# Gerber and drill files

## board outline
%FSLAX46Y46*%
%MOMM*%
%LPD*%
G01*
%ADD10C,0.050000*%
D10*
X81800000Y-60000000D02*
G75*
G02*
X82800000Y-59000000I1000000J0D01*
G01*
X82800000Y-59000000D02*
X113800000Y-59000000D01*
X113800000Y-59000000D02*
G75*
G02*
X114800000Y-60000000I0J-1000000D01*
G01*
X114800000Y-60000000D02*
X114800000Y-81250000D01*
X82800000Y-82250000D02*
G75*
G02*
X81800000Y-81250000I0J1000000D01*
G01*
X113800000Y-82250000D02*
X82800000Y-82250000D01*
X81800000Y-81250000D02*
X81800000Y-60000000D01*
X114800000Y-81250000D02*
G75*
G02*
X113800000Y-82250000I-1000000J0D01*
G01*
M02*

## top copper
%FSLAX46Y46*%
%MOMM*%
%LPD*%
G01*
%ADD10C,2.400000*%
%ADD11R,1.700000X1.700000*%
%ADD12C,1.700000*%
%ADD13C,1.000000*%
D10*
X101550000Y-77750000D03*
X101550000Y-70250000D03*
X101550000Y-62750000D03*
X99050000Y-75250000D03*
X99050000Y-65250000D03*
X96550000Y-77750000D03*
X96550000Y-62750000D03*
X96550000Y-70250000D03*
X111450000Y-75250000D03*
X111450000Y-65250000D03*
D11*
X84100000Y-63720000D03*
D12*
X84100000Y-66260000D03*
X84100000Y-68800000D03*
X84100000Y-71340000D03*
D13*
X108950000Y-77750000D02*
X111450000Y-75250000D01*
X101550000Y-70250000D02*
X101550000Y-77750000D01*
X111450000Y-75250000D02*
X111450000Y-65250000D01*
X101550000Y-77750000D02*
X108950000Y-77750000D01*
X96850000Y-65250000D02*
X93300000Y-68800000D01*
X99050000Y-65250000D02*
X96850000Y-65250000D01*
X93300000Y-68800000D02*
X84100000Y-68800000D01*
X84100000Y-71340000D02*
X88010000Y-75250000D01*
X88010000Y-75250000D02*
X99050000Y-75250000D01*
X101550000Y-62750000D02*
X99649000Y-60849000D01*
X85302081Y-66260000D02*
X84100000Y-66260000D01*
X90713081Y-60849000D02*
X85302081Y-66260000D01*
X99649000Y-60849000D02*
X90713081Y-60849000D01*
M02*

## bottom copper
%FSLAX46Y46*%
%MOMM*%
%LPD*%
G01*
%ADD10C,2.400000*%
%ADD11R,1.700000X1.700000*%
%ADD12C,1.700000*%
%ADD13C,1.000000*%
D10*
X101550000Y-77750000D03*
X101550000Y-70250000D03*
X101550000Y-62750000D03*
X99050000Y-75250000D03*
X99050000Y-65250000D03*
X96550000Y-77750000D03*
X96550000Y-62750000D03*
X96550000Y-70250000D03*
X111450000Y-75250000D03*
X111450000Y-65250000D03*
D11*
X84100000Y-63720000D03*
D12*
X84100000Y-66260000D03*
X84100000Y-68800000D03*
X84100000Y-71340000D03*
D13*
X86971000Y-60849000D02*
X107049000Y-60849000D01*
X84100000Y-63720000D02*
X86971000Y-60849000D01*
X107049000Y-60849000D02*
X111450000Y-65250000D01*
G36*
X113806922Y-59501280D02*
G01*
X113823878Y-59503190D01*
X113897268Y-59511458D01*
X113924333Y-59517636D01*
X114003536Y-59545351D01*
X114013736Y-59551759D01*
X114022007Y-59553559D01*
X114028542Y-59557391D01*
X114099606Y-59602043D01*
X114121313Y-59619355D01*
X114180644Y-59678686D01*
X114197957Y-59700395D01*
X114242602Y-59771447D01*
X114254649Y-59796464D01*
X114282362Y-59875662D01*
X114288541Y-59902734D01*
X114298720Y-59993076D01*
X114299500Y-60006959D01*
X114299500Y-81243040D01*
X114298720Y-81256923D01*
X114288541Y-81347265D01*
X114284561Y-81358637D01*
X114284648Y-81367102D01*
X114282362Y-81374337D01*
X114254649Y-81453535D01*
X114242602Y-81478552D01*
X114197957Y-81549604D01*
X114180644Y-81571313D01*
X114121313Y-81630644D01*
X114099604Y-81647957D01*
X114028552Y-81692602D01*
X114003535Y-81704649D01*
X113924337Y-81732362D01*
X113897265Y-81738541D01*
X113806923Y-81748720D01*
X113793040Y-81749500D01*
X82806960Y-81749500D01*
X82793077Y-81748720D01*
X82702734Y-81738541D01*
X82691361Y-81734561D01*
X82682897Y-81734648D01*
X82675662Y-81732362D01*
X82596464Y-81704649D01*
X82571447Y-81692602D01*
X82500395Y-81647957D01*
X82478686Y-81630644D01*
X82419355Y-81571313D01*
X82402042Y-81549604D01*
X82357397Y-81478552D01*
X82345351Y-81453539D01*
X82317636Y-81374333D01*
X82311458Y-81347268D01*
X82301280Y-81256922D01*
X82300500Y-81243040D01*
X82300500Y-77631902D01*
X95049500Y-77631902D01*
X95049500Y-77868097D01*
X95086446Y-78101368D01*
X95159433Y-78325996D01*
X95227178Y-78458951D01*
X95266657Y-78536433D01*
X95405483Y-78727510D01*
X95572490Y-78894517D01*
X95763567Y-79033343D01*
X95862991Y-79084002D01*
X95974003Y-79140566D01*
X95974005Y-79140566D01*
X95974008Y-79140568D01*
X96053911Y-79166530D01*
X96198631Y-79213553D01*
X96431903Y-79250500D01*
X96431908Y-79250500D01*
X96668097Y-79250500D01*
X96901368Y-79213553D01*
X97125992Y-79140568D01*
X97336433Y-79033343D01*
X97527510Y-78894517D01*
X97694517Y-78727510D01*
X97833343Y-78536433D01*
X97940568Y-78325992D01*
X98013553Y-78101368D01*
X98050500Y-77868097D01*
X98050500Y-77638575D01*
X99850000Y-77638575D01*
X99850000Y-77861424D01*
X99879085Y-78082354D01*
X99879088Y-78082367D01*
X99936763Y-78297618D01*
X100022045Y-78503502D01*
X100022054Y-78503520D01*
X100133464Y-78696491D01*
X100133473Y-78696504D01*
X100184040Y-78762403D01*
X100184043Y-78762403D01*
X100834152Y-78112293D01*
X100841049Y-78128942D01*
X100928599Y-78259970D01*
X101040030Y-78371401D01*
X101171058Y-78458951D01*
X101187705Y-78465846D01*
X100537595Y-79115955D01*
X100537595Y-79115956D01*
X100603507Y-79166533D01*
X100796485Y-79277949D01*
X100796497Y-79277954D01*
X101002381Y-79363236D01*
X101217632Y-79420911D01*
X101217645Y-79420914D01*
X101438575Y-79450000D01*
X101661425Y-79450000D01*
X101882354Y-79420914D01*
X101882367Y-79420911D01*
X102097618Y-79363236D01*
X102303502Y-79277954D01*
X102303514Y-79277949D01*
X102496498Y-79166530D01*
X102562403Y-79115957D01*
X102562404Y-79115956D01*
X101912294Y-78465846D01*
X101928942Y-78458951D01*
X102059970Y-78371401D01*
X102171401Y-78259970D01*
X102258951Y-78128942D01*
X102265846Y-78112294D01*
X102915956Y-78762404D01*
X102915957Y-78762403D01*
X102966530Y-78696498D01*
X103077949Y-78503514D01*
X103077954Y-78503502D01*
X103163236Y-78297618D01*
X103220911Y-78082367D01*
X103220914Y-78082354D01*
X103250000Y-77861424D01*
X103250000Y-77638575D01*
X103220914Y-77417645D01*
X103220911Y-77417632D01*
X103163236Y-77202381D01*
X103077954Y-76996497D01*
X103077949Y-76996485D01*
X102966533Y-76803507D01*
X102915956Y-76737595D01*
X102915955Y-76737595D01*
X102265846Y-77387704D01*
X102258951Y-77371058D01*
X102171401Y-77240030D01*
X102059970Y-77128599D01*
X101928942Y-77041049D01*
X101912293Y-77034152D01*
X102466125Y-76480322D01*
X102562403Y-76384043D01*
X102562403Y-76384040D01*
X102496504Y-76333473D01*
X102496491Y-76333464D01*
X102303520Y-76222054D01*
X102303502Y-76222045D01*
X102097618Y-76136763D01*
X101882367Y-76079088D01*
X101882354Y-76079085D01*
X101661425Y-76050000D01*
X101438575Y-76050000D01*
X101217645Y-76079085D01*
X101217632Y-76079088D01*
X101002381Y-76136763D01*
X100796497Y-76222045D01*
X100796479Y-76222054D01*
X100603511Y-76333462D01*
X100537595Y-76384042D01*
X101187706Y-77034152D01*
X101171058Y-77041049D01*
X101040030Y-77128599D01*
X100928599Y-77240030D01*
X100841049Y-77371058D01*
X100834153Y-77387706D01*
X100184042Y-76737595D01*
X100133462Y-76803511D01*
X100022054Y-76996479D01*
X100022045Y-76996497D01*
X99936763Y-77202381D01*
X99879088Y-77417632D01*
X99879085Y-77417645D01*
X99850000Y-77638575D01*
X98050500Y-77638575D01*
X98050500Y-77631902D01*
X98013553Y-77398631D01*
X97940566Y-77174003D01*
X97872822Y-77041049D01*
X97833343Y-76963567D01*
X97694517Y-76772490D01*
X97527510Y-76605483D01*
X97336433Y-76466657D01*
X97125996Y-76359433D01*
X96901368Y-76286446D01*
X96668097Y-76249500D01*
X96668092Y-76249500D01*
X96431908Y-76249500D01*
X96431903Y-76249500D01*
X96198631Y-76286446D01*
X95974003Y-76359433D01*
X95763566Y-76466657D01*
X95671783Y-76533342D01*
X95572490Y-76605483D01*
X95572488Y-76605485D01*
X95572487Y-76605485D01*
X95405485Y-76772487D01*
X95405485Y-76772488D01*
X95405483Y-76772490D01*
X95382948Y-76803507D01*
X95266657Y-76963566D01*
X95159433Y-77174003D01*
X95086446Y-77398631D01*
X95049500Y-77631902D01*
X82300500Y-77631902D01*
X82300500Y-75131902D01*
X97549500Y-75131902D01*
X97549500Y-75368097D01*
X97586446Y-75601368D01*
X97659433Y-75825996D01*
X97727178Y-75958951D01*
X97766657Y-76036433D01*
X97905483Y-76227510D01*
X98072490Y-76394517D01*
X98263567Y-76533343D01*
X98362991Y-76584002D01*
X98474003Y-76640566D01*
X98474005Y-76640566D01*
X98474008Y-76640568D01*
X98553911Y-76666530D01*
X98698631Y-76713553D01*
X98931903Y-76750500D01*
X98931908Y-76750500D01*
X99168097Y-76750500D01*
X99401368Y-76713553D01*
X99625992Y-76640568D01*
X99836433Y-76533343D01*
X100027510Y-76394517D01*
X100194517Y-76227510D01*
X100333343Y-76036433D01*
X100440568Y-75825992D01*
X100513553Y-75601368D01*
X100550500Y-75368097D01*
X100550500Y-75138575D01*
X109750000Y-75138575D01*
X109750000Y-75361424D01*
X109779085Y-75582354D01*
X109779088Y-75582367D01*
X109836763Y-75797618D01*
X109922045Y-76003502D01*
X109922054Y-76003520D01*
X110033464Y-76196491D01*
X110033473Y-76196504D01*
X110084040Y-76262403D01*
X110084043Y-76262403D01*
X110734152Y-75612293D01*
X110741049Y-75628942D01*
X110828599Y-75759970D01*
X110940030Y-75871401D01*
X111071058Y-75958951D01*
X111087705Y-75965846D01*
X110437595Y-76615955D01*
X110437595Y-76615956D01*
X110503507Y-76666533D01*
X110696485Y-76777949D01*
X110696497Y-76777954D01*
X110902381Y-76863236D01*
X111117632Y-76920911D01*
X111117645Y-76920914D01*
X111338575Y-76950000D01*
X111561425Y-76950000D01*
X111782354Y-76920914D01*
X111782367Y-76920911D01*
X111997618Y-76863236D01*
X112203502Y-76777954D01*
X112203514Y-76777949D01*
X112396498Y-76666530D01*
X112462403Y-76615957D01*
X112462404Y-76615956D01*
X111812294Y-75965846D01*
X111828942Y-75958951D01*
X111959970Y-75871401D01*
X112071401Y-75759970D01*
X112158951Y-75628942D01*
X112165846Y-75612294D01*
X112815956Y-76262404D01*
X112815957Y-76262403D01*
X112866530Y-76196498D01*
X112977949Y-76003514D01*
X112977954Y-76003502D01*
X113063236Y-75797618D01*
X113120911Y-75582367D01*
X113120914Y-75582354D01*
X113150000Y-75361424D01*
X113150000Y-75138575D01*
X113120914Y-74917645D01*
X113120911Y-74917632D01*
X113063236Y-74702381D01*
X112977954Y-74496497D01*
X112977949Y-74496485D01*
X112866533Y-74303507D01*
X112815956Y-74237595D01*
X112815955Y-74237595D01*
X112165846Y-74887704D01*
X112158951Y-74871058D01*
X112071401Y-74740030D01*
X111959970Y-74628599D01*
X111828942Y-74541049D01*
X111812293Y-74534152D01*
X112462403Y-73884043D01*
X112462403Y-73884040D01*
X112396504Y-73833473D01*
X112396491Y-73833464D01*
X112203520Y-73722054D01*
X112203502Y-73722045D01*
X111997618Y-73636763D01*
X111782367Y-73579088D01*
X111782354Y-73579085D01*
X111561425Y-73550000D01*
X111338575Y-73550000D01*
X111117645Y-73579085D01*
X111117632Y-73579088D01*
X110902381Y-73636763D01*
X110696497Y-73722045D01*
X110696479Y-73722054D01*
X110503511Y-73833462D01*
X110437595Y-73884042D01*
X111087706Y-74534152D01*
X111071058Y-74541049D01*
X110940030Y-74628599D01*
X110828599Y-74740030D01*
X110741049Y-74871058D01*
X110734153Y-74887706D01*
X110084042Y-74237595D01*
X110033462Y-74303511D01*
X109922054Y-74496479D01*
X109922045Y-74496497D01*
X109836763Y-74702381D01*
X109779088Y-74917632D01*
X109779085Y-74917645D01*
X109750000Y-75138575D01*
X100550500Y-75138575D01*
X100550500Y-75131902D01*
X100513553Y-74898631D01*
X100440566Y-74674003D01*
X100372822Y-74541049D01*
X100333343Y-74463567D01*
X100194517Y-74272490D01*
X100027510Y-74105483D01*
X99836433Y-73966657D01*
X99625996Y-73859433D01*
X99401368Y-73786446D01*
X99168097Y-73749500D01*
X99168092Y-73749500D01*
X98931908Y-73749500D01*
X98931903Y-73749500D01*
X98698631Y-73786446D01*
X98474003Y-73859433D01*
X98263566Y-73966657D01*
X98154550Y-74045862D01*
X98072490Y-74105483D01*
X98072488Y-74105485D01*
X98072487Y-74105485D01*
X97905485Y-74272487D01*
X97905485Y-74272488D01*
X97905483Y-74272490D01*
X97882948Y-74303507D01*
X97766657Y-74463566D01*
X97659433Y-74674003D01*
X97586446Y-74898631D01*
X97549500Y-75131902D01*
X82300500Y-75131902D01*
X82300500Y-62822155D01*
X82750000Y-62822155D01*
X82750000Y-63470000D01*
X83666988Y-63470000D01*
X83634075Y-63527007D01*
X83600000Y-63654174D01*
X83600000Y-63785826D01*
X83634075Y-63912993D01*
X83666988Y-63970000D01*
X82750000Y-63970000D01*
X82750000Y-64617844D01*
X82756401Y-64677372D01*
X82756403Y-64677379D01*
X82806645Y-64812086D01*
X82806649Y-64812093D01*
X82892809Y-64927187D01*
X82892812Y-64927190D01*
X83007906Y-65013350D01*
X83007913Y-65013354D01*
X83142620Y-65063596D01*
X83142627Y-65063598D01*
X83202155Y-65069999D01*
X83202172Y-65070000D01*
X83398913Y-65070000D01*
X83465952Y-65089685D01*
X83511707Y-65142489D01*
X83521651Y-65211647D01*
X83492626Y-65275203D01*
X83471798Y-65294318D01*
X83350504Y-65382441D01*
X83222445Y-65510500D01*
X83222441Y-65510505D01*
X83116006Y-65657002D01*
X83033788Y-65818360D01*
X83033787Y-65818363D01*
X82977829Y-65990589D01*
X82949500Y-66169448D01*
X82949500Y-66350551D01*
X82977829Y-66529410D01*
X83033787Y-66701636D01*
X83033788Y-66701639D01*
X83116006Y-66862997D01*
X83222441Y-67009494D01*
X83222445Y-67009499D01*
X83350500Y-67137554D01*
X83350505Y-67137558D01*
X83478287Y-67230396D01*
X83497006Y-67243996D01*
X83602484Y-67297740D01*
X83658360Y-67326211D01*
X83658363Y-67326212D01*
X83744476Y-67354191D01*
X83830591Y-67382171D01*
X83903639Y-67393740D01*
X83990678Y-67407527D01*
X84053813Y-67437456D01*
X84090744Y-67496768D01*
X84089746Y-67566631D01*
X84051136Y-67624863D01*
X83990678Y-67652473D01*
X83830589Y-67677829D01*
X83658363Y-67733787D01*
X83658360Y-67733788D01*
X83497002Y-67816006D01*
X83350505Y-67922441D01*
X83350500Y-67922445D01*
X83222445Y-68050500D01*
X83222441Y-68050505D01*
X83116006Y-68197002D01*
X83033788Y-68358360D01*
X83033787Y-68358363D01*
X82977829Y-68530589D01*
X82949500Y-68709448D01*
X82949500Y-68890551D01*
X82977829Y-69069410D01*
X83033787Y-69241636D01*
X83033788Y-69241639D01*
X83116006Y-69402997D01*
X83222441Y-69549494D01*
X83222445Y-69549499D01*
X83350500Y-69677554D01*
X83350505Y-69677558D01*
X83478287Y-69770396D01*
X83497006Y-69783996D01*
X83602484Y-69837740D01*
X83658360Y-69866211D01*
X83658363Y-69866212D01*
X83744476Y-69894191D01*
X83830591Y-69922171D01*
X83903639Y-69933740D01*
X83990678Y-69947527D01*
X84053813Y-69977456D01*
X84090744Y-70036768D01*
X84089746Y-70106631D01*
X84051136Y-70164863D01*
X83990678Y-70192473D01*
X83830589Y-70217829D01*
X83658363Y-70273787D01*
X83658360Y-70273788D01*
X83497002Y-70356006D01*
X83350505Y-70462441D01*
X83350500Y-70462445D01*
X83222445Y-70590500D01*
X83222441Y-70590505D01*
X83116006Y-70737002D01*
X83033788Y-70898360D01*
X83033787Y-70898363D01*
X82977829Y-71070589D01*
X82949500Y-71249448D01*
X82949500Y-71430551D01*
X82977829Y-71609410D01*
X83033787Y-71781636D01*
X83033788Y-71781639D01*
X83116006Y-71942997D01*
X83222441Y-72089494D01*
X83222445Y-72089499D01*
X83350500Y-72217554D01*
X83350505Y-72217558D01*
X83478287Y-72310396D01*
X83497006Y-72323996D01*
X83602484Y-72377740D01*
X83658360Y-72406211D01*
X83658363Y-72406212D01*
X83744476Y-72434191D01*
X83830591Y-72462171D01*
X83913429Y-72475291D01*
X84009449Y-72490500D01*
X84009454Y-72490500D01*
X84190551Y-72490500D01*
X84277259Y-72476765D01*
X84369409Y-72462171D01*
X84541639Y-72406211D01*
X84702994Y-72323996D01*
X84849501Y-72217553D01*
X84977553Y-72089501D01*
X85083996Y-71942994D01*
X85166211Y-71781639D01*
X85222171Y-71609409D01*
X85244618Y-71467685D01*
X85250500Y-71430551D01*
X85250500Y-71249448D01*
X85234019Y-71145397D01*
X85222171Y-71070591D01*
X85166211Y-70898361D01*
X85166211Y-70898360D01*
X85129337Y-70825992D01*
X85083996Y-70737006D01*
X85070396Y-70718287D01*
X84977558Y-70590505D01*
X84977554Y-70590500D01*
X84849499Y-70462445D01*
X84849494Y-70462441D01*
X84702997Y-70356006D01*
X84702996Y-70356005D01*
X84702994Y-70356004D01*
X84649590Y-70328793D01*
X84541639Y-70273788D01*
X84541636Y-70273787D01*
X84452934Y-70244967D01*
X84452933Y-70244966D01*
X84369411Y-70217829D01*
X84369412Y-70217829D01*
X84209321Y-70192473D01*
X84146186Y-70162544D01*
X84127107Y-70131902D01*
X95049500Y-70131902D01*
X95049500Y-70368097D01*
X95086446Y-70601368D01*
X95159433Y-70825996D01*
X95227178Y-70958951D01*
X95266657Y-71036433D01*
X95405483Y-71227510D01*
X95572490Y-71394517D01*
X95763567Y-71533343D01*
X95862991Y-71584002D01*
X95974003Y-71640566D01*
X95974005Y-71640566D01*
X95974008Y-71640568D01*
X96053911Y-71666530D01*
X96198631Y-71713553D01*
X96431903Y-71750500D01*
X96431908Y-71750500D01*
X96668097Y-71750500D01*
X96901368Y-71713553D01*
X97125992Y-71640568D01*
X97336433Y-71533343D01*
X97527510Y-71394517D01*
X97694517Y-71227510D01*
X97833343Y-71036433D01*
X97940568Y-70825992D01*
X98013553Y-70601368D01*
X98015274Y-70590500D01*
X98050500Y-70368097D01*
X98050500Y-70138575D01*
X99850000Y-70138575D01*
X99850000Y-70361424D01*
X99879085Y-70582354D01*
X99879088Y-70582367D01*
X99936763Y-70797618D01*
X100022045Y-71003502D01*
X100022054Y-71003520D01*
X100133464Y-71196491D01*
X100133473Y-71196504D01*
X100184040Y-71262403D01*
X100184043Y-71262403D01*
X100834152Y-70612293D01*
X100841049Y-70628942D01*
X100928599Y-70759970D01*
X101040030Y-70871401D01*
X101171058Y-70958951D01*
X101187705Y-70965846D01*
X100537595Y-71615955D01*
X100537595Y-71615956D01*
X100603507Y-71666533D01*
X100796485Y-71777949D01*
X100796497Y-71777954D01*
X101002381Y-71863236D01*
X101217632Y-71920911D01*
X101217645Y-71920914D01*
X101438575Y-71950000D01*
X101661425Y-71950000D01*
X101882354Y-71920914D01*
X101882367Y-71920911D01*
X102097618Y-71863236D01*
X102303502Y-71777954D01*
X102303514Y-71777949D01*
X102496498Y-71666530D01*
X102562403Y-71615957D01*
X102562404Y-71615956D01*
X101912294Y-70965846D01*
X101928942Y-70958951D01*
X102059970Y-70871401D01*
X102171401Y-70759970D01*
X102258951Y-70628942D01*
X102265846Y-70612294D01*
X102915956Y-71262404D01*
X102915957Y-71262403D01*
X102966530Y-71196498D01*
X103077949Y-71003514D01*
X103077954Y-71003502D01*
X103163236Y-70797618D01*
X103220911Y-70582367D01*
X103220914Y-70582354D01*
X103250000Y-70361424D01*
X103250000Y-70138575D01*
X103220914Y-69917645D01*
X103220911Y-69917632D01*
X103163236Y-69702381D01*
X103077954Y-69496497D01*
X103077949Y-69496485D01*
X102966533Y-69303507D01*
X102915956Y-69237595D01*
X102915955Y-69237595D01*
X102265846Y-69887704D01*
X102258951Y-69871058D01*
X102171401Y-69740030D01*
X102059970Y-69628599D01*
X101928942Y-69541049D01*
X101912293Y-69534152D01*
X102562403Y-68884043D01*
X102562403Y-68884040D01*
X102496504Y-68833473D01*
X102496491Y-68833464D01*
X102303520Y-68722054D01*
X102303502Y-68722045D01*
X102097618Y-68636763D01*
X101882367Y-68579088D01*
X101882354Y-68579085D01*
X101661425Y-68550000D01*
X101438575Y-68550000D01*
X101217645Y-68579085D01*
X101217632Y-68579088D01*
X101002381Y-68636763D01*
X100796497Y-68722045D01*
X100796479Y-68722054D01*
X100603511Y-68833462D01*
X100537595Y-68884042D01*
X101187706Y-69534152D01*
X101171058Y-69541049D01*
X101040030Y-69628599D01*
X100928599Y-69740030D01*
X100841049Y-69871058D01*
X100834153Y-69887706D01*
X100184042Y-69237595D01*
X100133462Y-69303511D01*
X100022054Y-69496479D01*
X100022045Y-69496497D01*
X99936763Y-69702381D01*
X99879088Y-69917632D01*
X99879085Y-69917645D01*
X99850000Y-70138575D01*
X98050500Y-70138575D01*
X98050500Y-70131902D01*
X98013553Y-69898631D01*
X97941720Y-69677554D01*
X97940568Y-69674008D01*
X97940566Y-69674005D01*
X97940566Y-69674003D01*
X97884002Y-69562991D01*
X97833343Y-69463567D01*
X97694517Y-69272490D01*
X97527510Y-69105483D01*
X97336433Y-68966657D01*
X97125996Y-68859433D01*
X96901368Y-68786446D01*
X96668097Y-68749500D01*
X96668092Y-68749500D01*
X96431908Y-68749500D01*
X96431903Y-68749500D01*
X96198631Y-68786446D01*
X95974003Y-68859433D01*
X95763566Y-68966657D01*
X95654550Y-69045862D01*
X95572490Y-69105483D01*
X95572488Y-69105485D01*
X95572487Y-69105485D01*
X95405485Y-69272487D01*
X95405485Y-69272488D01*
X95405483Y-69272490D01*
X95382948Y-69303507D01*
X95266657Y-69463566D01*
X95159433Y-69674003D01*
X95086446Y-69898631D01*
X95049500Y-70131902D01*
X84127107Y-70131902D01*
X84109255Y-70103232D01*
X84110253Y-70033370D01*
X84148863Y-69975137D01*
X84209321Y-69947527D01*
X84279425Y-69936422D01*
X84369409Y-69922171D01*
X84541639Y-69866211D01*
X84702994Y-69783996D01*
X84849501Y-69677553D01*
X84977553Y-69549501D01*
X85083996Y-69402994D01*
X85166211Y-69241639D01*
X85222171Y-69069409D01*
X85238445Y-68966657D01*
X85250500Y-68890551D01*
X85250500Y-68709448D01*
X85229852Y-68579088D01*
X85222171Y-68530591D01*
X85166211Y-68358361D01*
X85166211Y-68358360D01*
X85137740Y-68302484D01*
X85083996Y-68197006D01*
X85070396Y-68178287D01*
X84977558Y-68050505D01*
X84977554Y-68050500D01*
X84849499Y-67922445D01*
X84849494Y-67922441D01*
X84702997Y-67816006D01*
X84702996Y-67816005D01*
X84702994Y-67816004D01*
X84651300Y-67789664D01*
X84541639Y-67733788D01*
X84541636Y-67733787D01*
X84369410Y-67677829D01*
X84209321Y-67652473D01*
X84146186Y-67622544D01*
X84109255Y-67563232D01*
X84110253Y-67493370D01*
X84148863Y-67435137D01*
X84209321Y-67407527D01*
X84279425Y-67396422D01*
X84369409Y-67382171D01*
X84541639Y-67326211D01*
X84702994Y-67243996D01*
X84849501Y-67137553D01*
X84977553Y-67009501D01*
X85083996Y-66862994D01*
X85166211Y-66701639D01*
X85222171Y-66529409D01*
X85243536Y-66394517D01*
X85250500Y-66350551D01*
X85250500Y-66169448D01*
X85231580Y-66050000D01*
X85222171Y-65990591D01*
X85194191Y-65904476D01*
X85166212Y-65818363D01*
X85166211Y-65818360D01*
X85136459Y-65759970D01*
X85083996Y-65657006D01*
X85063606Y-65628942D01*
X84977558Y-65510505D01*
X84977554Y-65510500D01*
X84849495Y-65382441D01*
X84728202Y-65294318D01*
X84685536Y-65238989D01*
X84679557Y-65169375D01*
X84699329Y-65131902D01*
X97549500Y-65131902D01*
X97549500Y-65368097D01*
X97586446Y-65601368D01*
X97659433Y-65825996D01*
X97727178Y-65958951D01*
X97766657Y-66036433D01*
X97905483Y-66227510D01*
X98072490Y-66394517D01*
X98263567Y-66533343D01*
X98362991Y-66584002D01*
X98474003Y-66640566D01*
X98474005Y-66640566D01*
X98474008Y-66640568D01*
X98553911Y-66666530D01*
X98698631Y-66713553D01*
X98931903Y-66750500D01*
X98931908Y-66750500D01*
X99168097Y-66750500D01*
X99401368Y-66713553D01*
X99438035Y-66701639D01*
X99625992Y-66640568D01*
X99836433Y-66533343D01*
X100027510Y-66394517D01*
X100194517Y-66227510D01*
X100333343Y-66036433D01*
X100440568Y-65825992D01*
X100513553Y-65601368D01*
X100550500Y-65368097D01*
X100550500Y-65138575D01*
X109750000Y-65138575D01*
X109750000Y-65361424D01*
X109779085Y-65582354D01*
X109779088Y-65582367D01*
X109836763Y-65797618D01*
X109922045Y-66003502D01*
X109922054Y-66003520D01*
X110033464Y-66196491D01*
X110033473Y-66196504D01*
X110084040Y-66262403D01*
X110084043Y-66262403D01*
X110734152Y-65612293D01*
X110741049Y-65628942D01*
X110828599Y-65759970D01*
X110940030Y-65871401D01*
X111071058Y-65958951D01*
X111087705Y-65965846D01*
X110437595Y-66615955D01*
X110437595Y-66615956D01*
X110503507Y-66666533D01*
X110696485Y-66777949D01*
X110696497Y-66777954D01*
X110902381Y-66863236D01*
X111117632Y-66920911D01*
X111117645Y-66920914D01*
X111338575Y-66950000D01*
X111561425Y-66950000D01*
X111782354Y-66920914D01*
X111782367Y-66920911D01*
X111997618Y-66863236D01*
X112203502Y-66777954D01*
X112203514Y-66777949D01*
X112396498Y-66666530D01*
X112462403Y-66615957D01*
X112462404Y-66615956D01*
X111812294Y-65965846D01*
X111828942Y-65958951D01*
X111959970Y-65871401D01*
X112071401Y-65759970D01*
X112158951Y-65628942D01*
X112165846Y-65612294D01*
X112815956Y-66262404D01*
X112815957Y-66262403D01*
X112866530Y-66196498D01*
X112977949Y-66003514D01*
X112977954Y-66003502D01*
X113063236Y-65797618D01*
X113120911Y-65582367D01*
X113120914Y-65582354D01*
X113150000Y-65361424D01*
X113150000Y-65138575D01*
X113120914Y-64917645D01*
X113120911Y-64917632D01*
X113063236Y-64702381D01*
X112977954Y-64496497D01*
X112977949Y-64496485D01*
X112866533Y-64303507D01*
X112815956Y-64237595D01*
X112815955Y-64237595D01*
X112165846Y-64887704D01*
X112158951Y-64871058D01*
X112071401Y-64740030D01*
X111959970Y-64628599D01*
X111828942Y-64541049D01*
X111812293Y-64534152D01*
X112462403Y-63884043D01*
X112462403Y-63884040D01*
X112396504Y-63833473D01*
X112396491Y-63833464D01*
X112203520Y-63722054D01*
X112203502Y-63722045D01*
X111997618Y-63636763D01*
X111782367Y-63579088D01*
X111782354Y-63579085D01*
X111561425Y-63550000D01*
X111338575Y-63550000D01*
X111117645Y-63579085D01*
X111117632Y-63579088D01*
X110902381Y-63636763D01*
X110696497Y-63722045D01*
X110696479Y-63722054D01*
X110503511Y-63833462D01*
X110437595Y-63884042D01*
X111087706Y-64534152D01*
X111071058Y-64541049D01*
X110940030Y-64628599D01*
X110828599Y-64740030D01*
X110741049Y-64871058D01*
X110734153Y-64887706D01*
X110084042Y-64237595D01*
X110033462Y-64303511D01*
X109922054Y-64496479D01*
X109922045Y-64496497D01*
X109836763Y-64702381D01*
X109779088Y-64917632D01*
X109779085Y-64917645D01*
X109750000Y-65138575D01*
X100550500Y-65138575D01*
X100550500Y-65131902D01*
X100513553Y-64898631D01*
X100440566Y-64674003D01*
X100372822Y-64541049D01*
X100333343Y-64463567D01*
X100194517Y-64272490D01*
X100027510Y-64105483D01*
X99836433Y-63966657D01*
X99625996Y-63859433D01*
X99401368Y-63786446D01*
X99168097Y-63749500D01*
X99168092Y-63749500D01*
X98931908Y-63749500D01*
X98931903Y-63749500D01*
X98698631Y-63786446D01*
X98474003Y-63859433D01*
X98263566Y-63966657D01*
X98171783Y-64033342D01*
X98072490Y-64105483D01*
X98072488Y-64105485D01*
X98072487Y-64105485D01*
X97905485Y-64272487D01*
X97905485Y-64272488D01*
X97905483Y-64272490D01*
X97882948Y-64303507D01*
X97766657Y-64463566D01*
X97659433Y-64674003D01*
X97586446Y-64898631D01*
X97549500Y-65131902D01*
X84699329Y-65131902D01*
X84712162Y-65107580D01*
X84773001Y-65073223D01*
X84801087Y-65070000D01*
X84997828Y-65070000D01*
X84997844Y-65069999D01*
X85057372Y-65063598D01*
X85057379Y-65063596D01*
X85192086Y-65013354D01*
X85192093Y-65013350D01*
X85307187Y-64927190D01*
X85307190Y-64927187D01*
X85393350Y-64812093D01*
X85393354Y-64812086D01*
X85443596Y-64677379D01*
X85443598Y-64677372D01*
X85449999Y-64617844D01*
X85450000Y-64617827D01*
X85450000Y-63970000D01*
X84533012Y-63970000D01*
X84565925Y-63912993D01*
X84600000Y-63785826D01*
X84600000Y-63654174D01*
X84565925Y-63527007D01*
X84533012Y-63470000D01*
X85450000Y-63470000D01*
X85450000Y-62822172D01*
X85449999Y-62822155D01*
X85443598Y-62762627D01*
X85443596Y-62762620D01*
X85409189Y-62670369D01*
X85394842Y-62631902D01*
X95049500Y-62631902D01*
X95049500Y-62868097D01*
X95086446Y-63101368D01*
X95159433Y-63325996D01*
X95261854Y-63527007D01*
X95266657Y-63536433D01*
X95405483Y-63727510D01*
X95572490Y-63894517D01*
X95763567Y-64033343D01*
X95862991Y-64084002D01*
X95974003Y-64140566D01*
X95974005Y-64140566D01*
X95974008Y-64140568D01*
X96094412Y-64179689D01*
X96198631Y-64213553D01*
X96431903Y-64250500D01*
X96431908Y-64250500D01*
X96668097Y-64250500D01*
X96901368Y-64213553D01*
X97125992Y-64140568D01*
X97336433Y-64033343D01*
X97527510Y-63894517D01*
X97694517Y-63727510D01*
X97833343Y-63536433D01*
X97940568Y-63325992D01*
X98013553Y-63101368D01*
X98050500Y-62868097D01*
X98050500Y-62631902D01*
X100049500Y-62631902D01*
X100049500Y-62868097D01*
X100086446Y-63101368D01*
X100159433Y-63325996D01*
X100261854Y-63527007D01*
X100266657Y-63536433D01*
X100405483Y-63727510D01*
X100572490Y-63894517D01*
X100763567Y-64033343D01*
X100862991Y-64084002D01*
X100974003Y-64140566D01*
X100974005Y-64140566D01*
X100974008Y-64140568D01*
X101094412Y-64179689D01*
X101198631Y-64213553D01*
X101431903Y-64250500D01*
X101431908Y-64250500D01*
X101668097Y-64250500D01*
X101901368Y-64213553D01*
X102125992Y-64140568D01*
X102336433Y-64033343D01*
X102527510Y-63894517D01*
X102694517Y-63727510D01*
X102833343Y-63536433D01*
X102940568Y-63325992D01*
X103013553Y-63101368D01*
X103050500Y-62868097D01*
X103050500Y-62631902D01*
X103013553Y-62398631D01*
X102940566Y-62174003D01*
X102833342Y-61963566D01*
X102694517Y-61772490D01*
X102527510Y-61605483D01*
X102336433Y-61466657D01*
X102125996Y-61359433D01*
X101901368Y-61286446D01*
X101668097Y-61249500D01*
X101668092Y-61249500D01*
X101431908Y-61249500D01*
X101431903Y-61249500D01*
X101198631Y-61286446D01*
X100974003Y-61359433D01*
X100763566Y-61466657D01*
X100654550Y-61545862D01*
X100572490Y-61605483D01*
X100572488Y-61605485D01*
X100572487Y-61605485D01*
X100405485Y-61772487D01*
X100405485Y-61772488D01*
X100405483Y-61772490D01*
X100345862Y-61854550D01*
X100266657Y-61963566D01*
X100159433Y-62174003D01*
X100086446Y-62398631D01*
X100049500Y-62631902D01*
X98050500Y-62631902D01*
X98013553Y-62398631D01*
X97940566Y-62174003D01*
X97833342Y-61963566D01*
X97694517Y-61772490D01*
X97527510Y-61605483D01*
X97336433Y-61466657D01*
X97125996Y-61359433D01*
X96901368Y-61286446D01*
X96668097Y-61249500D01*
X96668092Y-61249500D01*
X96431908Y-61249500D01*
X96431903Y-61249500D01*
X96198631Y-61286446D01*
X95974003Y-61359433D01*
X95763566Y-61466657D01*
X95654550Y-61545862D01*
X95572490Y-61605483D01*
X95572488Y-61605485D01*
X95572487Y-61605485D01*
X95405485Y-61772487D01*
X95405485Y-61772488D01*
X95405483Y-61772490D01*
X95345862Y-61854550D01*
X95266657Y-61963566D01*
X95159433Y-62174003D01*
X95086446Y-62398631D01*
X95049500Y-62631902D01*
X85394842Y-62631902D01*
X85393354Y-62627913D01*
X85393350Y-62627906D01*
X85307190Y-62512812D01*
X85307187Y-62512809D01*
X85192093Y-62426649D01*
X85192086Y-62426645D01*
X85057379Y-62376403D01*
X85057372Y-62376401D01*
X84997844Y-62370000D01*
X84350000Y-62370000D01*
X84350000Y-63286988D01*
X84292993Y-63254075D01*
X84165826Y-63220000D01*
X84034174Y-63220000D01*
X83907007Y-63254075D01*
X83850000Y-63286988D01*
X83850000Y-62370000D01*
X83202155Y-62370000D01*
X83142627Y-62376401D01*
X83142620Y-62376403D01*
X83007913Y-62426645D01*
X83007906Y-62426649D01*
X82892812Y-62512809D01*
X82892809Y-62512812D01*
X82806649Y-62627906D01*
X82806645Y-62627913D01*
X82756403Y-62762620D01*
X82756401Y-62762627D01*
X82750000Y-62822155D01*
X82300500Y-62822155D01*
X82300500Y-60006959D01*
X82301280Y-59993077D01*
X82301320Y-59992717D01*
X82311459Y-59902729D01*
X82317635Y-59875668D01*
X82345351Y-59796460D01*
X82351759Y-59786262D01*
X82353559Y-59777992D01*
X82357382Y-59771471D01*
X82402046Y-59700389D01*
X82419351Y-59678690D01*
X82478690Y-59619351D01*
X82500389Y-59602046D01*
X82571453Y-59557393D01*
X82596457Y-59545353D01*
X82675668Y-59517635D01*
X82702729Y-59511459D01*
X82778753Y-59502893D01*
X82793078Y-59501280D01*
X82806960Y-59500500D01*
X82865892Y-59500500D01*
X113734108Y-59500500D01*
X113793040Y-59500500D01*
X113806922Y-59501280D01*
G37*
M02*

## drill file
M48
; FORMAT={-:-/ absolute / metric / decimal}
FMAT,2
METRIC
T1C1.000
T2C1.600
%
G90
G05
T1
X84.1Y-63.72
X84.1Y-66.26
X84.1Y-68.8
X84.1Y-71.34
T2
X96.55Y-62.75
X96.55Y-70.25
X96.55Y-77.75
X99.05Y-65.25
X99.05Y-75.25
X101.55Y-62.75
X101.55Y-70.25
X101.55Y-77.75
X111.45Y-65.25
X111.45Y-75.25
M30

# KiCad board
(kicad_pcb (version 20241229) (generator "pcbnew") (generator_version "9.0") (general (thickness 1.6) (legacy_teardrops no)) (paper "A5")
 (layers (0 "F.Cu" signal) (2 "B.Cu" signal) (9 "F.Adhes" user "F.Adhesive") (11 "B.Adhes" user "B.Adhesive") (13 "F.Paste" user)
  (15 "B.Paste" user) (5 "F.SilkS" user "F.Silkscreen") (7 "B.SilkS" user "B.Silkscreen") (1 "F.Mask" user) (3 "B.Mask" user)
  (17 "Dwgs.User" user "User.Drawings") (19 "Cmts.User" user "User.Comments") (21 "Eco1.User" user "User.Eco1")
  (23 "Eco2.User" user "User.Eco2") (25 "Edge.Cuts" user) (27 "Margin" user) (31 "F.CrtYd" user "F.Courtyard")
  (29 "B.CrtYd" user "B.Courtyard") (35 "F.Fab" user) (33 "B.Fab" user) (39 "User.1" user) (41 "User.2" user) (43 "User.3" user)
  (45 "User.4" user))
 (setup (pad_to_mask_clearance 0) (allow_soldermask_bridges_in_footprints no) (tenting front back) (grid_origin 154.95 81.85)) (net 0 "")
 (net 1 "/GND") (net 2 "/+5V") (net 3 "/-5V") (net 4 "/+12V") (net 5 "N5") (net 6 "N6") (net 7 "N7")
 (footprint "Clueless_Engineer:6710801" (layer "F.Cu") (at 101.55 77.75 -90)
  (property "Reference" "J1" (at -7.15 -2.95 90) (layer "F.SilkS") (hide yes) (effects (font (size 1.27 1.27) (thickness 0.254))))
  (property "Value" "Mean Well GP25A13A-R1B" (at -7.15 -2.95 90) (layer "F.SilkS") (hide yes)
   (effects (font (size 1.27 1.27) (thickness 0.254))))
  (pad "1" thru_hole circle (at 0 0 270) (size 2.4 2.4) (drill 1.6) (layers "*.Cu" "*.Mask") (remove_unused_layers no) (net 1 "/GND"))
  (pad "2" thru_hole circle (at -7.5 0 270) (size 2.4 2.4) (drill 1.6) (layers "*.Cu" "*.Mask") (remove_unused_layers no) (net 1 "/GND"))
  (pad "3" thru_hole circle (at -15 0 270) (size 2.4 2.4) (drill 1.6) (layers "*.Cu" "*.Mask") (remove_unused_layers no) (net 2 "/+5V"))
  (pad "4" thru_hole circle (at -2.5 2.5 270) (size 2.4 2.4) (drill 1.6) (layers "*.Cu" "*.Mask") (remove_unused_layers no) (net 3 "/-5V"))
  (pad "5" thru_hole circle (at -12.5 2.5 270) (size 2.4 2.4) (drill 1.6) (layers "*.Cu" "*.Mask") (remove_unused_layers no) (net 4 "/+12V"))
  (pad "6" thru_hole circle (at 0 5 270) (size 2.4 2.4) (drill 1.6) (layers "*.Cu" "*.Mask") (remove_unused_layers no) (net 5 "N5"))
  (pad "7" thru_hole circle (at -15 5 270) (size 2.4 2.4) (drill 1.6) (layers "*.Cu" "*.Mask") (remove_unused_layers no) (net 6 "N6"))
  (pad "8" thru_hole circle (at -7.5 5 270) (size 2.4 2.4) (drill 1.6) (layers "*.Cu" "*.Mask") (remove_unused_layers no) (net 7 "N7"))
  (pad "MH1" thru_hole circle (at -2.5 -9.9 270) (size 2.4 2.4) (drill 1.6) (layers "*.Cu" "*.Mask") (remove_unused_layers no)
   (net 1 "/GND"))
  (pad "MH2" thru_hole circle (at -12.5 -9.9 270) (size 2.4 2.4) (drill 1.6) (layers "*.Cu" "*.Mask") (remove_unused_layers no)
   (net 1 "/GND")))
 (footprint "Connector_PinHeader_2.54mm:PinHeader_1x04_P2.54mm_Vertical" (layer "F.Cu") (at 84.1 63.72)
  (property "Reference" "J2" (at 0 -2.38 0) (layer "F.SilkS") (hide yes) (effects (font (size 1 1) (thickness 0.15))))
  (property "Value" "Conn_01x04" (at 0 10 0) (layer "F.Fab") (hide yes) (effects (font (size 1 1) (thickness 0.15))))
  (pad "1" thru_hole rect (at 0 0) (size 1.7 1.7) (drill 1) (layers "*.Cu" "*.Mask") (remove_unused_layers no) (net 1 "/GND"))
  (pad "2" thru_hole circle (at 0 2.54) (size 1.7 1.7) (drill 1) (layers "*.Cu" "*.Mask") (remove_unused_layers no) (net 2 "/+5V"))
  (pad "3" thru_hole circle (at 0 5.08) (size 1.7 1.7) (drill 1) (layers "*.Cu" "*.Mask") (remove_unused_layers no) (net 4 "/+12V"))
  (pad "4" thru_hole circle (at 0 7.62) (size 1.7 1.7) (drill 1) (layers "*.Cu" "*.Mask") (remove_unused_layers no) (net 3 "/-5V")))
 (gr_arc (start 81.8 60) (mid 82.092893 59.292893) (end 82.8 59) (stroke (width 0.05) (type default)) (layer "Edge.Cuts"))
 (gr_line (start 82.8 59) (end 113.8 59) (stroke (width 0.05) (type default)) (layer "Edge.Cuts"))
 (gr_arc (start 113.8 59) (mid 114.507107 59.292893) (end 114.8 60) (stroke (width 0.05) (type default)) (layer "Edge.Cuts"))
 (gr_line (start 114.8 60) (end 114.8 81.25) (stroke (width 0.05) (type default)) (layer "Edge.Cuts"))
 (gr_arc (start 82.8 82.25) (mid 82.092893 81.957107) (end 81.8 81.25) (stroke (width 0.05) (type default)) (layer "Edge.Cuts"))
 (gr_line (start 113.8 82.25) (end 82.8 82.25) (stroke (width 0.05) (type default)) (layer "Edge.Cuts"))
 (gr_line (start 81.8 81.25) (end 81.8 60) (stroke (width 0.05) (type default)) (layer "Edge.Cuts"))
 (gr_arc (start 114.8 81.25) (mid 114.507107 81.957107) (end 113.8 82.25) (stroke (width 0.05) (type default)) (layer "Edge.Cuts"))
 (segment (start 108.95 77.75) (end 111.45 75.25) (width 1) (layer "F.Cu") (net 1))
 (segment (start 101.55 70.25) (end 101.55 77.75) (width 1) (layer "F.Cu") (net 1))
 (segment (start 111.45 75.25) (end 111.45 65.25) (width 1) (layer "F.Cu") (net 1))
 (segment (start 101.55 77.75) (end 108.95 77.75) (width 1) (layer "F.Cu") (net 1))
 (segment (start 86.971 60.849) (end 107.049 60.849) (width 1) (layer "B.Cu") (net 1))
 (segment (start 84.1 63.72) (end 86.971 60.849) (width 1) (layer "B.Cu") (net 1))
 (segment (start 107.049 60.849) (end 111.45 65.25) (width 1) (layer "B.Cu") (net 1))
 (segment (start 96.85 65.25) (end 93.3 68.8) (width 1) (layer "F.Cu") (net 4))
 (segment (start 99.05 65.25) (end 96.85 65.25) (width 1) (layer "F.Cu") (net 4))
 (segment (start 93.3 68.8) (end 84.1 68.8) (width 1) (layer "F.Cu") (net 4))
 (segment (start 84.1 71.34) (end 88.01 75.25) (width 1) (layer "F.Cu") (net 3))
 (segment (start 88.01 75.25) (end 99.05 75.25) (width 1) (layer "F.Cu") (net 3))
 (segment (start 101.55 62.75) (end 99.649 60.849) (width 1) (layer "F.Cu") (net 2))
 (segment (start 85.302081 66.26) (end 84.1 66.26) (width 1) (layer "F.Cu") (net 2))
 (segment (start 90.713081 60.849) (end 85.302081 66.26) (width 1) (layer "F.Cu") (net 2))
 (segment (start 99.649 60.849) (end 90.713081 60.849) (width 1) (layer "F.Cu") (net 2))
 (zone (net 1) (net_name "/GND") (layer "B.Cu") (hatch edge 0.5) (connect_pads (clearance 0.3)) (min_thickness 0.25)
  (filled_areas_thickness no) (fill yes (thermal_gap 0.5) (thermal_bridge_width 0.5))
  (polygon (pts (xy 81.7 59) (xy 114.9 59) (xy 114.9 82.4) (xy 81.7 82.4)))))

